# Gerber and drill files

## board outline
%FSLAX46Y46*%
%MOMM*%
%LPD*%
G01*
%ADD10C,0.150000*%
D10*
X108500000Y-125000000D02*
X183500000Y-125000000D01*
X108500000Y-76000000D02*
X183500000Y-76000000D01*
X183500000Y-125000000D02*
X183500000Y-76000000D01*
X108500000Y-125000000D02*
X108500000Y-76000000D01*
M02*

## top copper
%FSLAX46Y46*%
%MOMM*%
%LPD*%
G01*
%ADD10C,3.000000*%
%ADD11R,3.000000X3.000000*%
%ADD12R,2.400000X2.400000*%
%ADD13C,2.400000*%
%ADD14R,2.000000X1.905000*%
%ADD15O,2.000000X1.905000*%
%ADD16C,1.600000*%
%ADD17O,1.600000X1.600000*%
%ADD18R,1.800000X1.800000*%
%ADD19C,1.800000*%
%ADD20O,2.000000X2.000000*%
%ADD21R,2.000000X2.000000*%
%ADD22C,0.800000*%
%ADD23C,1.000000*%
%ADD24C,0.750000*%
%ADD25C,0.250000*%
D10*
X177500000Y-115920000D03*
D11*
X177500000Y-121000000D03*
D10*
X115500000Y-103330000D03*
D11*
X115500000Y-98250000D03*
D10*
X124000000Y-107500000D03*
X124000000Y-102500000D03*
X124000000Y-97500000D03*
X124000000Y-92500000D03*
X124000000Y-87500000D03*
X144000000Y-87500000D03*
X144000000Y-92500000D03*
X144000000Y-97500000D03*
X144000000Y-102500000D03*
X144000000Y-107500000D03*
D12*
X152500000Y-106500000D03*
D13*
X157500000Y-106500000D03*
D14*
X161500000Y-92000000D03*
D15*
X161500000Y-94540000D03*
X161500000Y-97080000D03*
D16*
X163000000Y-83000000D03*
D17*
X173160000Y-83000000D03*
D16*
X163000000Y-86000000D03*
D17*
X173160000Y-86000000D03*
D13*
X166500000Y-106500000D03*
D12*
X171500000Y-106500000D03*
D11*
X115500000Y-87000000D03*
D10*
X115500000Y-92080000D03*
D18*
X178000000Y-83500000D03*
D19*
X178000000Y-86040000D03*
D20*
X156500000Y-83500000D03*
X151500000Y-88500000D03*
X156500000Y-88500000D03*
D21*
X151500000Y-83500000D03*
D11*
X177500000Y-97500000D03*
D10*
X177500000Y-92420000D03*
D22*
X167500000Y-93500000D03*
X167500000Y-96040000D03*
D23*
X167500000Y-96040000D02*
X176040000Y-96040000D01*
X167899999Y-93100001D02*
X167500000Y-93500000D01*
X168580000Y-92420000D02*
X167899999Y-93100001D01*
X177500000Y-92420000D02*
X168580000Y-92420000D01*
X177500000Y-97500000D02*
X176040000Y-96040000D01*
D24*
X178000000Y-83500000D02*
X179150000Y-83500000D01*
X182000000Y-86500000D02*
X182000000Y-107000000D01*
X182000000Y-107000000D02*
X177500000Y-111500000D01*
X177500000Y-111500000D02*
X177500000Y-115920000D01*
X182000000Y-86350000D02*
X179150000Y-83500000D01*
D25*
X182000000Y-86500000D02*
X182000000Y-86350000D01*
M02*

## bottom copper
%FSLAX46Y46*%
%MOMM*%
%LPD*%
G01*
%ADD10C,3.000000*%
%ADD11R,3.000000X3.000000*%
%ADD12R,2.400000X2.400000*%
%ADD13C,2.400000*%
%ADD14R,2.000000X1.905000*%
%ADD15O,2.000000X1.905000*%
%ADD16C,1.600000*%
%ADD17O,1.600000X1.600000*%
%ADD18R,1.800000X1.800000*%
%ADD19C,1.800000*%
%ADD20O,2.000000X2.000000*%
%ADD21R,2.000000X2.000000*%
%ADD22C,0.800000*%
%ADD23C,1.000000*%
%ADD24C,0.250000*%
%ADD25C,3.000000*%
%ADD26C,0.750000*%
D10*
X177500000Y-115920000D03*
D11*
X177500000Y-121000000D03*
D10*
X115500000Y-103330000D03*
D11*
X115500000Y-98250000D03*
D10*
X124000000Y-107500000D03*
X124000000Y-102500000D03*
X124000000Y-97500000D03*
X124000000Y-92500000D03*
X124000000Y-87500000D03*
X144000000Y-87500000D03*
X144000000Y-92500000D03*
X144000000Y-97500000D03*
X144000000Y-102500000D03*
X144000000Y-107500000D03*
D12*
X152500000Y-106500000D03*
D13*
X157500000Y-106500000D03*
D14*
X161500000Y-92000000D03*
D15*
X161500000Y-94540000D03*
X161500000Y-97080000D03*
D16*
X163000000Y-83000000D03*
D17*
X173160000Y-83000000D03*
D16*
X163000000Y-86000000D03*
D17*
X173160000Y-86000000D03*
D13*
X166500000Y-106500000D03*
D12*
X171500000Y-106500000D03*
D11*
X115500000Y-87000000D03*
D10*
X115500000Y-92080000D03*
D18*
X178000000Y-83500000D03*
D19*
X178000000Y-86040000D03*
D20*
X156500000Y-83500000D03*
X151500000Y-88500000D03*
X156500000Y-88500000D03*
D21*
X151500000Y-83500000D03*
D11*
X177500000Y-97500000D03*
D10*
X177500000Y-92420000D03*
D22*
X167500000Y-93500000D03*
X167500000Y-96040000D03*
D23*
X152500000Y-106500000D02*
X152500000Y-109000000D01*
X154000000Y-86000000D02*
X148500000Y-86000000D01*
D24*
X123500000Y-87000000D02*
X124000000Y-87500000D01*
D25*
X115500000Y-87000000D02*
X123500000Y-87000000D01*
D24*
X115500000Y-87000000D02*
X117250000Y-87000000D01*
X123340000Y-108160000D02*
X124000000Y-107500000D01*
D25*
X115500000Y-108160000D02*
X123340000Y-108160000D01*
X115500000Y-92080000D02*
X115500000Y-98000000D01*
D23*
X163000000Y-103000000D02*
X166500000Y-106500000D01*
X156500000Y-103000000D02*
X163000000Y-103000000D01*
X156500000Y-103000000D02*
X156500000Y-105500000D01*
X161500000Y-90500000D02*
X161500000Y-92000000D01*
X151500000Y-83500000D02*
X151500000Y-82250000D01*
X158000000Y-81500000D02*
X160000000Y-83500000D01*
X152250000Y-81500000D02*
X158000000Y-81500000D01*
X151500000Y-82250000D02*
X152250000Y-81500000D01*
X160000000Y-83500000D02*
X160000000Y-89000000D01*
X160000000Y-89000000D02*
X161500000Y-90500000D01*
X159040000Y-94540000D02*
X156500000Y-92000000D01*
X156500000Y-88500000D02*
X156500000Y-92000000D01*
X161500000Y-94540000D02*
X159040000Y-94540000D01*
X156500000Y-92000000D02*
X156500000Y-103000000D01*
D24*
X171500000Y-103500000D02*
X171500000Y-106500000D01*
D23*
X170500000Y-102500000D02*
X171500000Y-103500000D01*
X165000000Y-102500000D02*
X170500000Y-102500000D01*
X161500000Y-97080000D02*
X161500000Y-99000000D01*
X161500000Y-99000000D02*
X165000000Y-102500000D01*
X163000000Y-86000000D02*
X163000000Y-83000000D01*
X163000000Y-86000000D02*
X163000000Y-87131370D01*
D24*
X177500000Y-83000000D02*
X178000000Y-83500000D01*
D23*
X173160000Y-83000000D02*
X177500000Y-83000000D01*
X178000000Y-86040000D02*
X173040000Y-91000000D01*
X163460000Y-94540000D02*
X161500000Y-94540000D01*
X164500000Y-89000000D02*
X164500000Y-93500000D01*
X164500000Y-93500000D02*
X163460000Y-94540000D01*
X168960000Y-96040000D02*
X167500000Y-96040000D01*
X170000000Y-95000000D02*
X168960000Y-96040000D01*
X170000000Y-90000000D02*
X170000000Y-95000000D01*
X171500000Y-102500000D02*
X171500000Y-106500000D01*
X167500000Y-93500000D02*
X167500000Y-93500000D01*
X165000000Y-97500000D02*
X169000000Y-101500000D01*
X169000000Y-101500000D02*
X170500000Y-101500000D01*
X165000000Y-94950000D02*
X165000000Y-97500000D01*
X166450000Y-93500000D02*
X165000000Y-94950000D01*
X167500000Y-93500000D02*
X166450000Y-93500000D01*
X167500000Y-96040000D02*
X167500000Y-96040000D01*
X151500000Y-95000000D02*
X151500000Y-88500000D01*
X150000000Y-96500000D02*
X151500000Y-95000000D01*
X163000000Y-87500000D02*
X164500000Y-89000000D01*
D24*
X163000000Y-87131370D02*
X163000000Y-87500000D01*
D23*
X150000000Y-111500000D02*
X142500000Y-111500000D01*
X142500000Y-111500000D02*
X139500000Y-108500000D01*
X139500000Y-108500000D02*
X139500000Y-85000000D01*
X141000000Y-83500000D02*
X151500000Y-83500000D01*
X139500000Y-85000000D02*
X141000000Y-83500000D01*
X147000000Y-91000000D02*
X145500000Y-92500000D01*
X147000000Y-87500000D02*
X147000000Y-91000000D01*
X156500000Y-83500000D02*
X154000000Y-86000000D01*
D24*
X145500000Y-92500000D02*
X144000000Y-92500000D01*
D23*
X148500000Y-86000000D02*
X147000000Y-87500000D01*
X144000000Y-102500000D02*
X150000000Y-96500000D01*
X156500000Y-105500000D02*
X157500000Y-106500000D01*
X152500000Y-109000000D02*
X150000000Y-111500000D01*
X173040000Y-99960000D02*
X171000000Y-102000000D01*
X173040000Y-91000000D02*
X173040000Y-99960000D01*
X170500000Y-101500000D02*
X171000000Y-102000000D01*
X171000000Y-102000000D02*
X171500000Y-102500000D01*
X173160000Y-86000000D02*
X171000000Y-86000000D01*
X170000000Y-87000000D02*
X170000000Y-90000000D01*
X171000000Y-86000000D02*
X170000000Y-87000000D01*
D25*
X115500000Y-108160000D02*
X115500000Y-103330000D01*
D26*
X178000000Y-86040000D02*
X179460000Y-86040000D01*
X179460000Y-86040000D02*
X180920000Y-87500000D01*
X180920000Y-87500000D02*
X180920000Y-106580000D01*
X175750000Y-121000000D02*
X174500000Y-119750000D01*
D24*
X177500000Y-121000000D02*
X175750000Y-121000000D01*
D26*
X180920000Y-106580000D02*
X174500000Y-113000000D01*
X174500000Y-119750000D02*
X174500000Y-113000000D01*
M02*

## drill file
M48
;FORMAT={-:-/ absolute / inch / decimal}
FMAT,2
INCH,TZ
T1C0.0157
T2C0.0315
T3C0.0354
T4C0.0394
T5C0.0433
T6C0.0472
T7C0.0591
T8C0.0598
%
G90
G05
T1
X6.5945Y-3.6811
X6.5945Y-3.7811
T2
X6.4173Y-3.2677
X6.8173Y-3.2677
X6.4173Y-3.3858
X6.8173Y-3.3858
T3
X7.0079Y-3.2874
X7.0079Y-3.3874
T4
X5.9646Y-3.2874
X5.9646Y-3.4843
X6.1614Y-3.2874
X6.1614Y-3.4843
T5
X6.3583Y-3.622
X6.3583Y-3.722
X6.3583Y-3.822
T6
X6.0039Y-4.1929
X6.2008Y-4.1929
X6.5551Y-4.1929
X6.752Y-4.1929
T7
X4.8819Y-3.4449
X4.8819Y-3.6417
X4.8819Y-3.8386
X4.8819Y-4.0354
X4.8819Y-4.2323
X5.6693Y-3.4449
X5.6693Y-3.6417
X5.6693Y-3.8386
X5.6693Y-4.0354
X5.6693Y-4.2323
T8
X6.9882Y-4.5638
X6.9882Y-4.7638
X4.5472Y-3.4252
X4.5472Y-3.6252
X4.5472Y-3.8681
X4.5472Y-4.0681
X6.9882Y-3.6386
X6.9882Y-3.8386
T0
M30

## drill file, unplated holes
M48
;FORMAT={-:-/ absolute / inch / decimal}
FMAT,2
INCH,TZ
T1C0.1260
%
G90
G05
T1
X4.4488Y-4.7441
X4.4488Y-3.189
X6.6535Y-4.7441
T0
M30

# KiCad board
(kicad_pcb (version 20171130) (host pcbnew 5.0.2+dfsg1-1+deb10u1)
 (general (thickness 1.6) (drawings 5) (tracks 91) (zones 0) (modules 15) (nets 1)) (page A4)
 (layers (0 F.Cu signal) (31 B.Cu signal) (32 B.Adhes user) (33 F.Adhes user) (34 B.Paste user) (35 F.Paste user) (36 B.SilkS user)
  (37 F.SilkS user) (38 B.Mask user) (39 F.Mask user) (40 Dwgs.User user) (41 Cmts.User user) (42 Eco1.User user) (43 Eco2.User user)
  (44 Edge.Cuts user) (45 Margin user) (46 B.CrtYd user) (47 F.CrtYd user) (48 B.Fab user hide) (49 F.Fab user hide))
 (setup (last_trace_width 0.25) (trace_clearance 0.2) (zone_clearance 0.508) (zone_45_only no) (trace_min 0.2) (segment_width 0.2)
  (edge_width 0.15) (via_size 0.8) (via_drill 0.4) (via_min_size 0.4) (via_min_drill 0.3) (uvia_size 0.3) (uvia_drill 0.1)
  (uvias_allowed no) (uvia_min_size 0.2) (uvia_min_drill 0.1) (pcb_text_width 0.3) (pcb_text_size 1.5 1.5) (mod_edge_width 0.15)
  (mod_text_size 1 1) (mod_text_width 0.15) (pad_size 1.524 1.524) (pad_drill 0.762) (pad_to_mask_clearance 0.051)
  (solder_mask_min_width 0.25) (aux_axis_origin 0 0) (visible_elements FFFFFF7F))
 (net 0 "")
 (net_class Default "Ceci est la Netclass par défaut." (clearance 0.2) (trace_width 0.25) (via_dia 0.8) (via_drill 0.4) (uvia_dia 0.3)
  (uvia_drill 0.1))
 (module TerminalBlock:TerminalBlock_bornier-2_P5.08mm (layer F.Cu) (at 177.5 121 90)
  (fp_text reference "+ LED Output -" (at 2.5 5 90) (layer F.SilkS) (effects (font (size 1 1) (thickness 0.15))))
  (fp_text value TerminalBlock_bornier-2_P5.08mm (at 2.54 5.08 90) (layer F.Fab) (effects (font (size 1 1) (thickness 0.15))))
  (pad 2 thru_hole circle (at 5.08 0 90) (size 3 3) (drill 1.52) (layers *.Cu *.Mask))
  (pad 1 thru_hole rect (at 0 0 90) (size 3 3) (drill 1.52) (layers *.Cu *.Mask)))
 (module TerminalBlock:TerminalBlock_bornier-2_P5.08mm (layer F.Cu) (at 115.5 98.25 270)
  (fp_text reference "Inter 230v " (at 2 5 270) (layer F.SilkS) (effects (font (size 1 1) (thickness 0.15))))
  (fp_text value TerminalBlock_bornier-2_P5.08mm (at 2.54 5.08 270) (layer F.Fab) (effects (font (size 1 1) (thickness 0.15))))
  (pad 2 thru_hole circle (at 5.08 0 270) (size 3 3) (drill 1.52) (layers *.Cu *.Mask))
  (pad 1 thru_hole rect (at 0 0 270) (size 3 3) (drill 1.52) (layers *.Cu *.Mask)))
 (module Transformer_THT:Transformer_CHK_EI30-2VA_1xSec (layer F.Cu) (at 124 107.5)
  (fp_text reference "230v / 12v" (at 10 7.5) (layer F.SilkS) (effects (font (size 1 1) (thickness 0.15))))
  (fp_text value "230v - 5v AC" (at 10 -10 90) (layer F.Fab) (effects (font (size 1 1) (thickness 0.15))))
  (pad 1 thru_hole circle (at 0 0) (size 3 3) (drill 1.5) (layers *.Cu *.Mask))
  (pad 2 thru_hole circle (at 0 -5) (size 3 3) (drill 1.5) (layers *.Cu *.Mask))
  (pad 3 thru_hole circle (at 0 -10) (size 3 3) (drill 1.5) (layers *.Cu *.Mask))
  (pad 4 thru_hole circle (at 0 -15) (size 3 3) (drill 1.5) (layers *.Cu *.Mask))
  (pad 5 thru_hole circle (at 0 -20) (size 3 3) (drill 1.5) (layers *.Cu *.Mask))
  (pad 6 thru_hole circle (at 20 -20) (size 3 3) (drill 1.5) (layers *.Cu *.Mask))
  (pad 7 thru_hole circle (at 20 -15) (size 3 3) (drill 1.5) (layers *.Cu *.Mask))
  (pad 8 thru_hole circle (at 20 -10) (size 3 3) (drill 1.5) (layers *.Cu *.Mask))
  (pad 9 thru_hole circle (at 20 -5) (size 3 3) (drill 1.5) (layers *.Cu *.Mask))
  (pad 10 thru_hole circle (at 20 0) (size 3 3) (drill 1.5) (layers *.Cu *.Mask)))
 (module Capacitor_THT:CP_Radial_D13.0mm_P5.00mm (layer F.Cu) (at 152.5 106.5)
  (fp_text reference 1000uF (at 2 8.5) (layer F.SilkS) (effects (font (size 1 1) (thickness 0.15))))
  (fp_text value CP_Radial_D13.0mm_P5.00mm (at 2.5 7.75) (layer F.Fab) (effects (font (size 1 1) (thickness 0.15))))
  (pad 1 thru_hole rect (at 0 0) (size 2.4 2.4) (drill 1.2) (layers *.Cu *.Mask))
  (pad 2 thru_hole circle (at 5 0) (size 2.4 2.4) (drill 1.2) (layers *.Cu *.Mask)))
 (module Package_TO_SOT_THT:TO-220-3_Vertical (layer F.Cu) (at 161.5 92 270)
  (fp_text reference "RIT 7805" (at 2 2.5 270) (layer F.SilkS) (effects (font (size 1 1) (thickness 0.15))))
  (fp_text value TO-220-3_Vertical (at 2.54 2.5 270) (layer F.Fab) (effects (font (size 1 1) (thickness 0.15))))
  (pad 1 thru_hole rect (at 0 0 270) (size 1.905 2) (drill 1.1) (layers *.Cu *.Mask))
  (pad 2 thru_hole oval (at 2.54 0 270) (size 1.905 2) (drill 1.1) (layers *.Cu *.Mask))
  (pad 3 thru_hole oval (at 5.08 0 270) (size 1.905 2) (drill 1.1) (layers *.Cu *.Mask)))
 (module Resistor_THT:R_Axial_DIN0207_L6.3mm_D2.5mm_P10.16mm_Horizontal (layer F.Cu) (at 163 83)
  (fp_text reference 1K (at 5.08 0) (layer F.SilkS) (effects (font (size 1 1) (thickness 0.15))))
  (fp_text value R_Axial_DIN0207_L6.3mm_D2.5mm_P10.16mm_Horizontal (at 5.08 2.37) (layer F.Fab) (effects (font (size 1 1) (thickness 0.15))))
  (pad 1 thru_hole circle (at 0 0) (size 1.6 1.6) (drill 0.8) (layers *.Cu *.Mask))
  (pad 2 thru_hole oval (at 10.16 0) (size 1.6 1.6) (drill 0.8) (layers *.Cu *.Mask)))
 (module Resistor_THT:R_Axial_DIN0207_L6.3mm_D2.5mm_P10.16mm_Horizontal (layer F.Cu) (at 163 86)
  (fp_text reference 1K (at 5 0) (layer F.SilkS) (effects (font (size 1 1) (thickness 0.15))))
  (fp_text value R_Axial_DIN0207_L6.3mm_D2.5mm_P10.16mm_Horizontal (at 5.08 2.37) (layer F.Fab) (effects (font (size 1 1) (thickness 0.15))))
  (pad 1 thru_hole circle (at 0 0) (size 1.6 1.6) (drill 0.8) (layers *.Cu *.Mask))
  (pad 2 thru_hole oval (at 10.16 0) (size 1.6 1.6) (drill 0.8) (layers *.Cu *.Mask)))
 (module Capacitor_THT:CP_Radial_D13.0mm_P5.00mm (layer F.Cu) (at 171.5 106.5 180)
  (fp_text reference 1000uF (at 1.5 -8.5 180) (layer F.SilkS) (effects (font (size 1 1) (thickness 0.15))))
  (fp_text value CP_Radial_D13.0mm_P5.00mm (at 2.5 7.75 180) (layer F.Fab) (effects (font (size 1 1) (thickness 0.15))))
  (pad 2 thru_hole circle (at 5 0 180) (size 2.4 2.4) (drill 1.2) (layers *.Cu *.Mask))
  (pad 1 thru_hole rect (at 0 0 180) (size 2.4 2.4) (drill 1.2) (layers *.Cu *.Mask)))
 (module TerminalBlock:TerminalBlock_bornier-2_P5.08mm (layer F.Cu) (at 115.5 87 270)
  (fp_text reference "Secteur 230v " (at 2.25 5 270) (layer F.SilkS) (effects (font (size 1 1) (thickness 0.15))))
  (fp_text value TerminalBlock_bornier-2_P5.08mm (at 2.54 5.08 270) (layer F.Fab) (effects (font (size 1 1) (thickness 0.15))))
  (pad 1 thru_hole rect (at 0 0 270) (size 3 3) (drill 1.52) (layers *.Cu *.Mask))
  (pad 2 thru_hole circle (at 5.08 0 270) (size 3 3) (drill 1.52) (layers *.Cu *.Mask)))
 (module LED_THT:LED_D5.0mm (layer F.Cu) (at 178 83.5 270)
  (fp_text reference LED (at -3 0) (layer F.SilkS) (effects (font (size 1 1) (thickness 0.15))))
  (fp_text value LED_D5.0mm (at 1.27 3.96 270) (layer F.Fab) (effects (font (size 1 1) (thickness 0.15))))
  (pad 1 thru_hole rect (at 0 0 270) (size 1.8 1.8) (drill 0.9) (layers *.Cu *.Mask))
  (pad 2 thru_hole circle (at 2.54 0 270) (size 1.8 1.8) (drill 0.9) (layers *.Cu *.Mask)))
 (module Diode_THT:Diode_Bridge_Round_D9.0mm (layer F.Cu) (at 151.5 83.5)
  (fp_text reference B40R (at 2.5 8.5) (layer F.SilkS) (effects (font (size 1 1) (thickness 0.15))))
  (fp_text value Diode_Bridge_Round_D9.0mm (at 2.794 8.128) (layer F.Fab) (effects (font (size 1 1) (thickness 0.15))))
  (pad 4 thru_hole oval (at 5 0) (size 2 2) (drill 1) (layers *.Cu *.Mask))
  (pad 2 thru_hole oval (at 0 5) (size 2 2) (drill 1) (layers *.Cu *.Mask))
  (pad 3 thru_hole oval (at 5 5) (size 2 2) (drill 1) (layers *.Cu *.Mask))
  (pad 1 thru_hole rect (at 0 0) (size 2 2) (drill 1) (layers *.Cu *.Mask)))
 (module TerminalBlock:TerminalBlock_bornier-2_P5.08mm (layer F.Cu) (at 177.5 97.5 90)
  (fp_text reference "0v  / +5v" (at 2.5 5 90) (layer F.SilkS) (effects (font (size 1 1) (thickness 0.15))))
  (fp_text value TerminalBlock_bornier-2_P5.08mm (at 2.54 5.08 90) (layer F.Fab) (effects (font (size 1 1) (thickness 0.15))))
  (pad 1 thru_hole rect (at 0 0 90) (size 3 3) (drill 1.52) (layers *.Cu *.Mask))
  (pad 2 thru_hole circle (at 5.08 0 90) (size 3 3) (drill 1.52) (layers *.Cu *.Mask)))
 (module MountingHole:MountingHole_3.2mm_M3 (layer F.Cu) (at 113 120.5)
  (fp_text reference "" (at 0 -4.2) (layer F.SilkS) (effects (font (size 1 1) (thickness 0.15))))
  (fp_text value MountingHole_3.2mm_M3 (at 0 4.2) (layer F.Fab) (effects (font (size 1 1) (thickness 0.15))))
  (pad 1 np_thru_hole circle (at 0 0) (size 3.2 3.2) (drill 3.2) (layers *.Cu *.Mask)))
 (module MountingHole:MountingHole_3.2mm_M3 (layer F.Cu) (at 113 81)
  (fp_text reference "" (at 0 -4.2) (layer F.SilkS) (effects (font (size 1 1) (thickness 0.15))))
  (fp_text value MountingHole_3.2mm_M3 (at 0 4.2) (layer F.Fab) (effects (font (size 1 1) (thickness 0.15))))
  (pad 1 np_thru_hole circle (at 0 0) (size 3.2 3.2) (drill 3.2) (layers *.Cu *.Mask)))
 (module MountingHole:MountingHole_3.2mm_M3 (layer F.Cu) (at 169 120.5)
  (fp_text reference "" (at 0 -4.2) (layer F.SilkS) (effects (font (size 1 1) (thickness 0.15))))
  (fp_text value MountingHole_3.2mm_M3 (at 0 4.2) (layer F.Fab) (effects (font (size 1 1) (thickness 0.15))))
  (pad 1 np_thru_hole circle (at 0 0) (size 3.2 3.2) (drill 3.2) (layers *.Cu *.Mask)))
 (gr_line (start 108.5 125) (end 183.5 125) (layer Edge.Cuts) (width 0.15))
 (gr_line (start 108.5 76) (end 183.5 76) (layer Edge.Cuts) (width 0.15))
 (gr_line (start 183.5 125) (end 183.5 76) (layer Edge.Cuts) (width 0.15))
 (gr_line (start 108.5 125) (end 108.5 76) (layer Edge.Cuts) (width 0.15))
 (segment (start 152.5 106.5) (end 152.5 109) (width 1) (layer B.Cu) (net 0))
 (segment (start 154 86) (end 148.5 86) (width 1) (layer B.Cu) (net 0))
 (segment (start 123.5 87) (end 124 87.5) (width 0.25) (layer B.Cu) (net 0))
 (segment (start 115.5 87) (end 123.5 87) (width 3) (layer B.Cu) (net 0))
 (segment (start 115.5 87) (end 117.25 87) (width 0.25) (layer B.Cu) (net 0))
 (segment (start 123.34 108.16) (end 124 107.5) (width 0.25) (layer B.Cu) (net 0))
 (segment (start 115.5 108.16) (end 123.34 108.16) (width 3) (layer B.Cu) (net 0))
 (segment (start 115.5 92.08) (end 115.5 98) (width 3) (layer B.Cu) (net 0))
 (segment (start 163 103) (end 166.5 106.5) (width 1) (layer B.Cu) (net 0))
 (segment (start 156.5 103) (end 163 103) (width 1) (layer B.Cu) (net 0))
 (segment (start 156.5 103) (end 156.5 105.5) (width 1) (layer B.Cu) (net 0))
 (segment (start 161.5 90.5) (end 161.5 92) (width 1) (layer B.Cu) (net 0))
 (segment (start 151.5 83.5) (end 151.5 82.25) (width 1) (layer B.Cu) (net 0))
 (segment (start 158 81.5) (end 160 83.5) (width 1) (layer B.Cu) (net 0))
 (segment (start 152.25 81.5) (end 158 81.5) (width 1) (layer B.Cu) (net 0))
 (segment (start 151.5 82.25) (end 152.25 81.5) (width 1) (layer B.Cu) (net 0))
 (segment (start 160 83.5) (end 160 89) (width 1) (layer B.Cu) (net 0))
 (segment (start 160 89) (end 161.5 90.5) (width 1) (layer B.Cu) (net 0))
 (segment (start 159.04 94.54) (end 156.5 92) (width 1) (layer B.Cu) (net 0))
 (segment (start 156.5 88.5) (end 156.5 92) (width 1) (layer B.Cu) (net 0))
 (segment (start 161.5 94.54) (end 159.04 94.54) (width 1) (layer B.Cu) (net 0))
 (segment (start 156.5 92) (end 156.5 103) (width 1) (layer B.Cu) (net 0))
 (segment (start 171.5 103.5) (end 171.5 106.5) (width 0.25) (layer B.Cu) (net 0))
 (segment (start 170.5 102.5) (end 171.5 103.5) (width 1) (layer B.Cu) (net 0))
 (segment (start 165 102.5) (end 170.5 102.5) (width 1) (layer B.Cu) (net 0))
 (segment (start 161.5 97.08) (end 161.5 99) (width 1) (layer B.Cu) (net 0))
 (segment (start 161.5 99) (end 165 102.5) (width 1) (layer B.Cu) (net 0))
 (segment (start 163 86) (end 163 83) (width 1) (layer B.Cu) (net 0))
 (segment (start 163 86) (end 163 87.13137) (width 1) (layer B.Cu) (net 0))
 (segment (start 177.5 83) (end 178 83.5) (width 0.25) (layer B.Cu) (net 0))
 (segment (start 173.16 83) (end 177.5 83) (width 1) (layer B.Cu) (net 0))
 (segment (start 178 86.04) (end 173.04 91) (width 1) (layer B.Cu) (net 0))
 (segment (start 163.46 94.54) (end 161.5 94.54) (width 1) (layer B.Cu) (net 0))
 (segment (start 164.5 89) (end 164.5 93.5) (width 1) (layer B.Cu) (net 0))
 (segment (start 164.5 93.5) (end 163.46 94.54) (width 1) (layer B.Cu) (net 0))
 (segment (start 168.96 96.04) (end 167.5 96.04) (width 1) (layer B.Cu) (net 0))
 (segment (start 170 95) (end 168.96 96.04) (width 1) (layer B.Cu) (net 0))
 (segment (start 170 90) (end 170 95) (width 1) (layer B.Cu) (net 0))
 (segment (start 171.5 102.5) (end 171.5 106.5) (width 1) (layer B.Cu) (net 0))
 (segment (start 167.5 93.5) (end 167.5 93.5) (width 1) (layer B.Cu) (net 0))
 (segment (start 165 97.5) (end 169 101.5) (width 1) (layer B.Cu) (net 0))
 (segment (start 169 101.5) (end 170.5 101.5) (width 1) (layer B.Cu) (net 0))
 (segment (start 165 94.95) (end 165 97.5) (width 1) (layer B.Cu) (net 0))
 (segment (start 166.45 93.5) (end 165 94.95) (width 1) (layer B.Cu) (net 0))
 (segment (start 167.5 93.5) (end 166.45 93.5) (width 1) (layer B.Cu) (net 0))
 (via (at 167.5 93.5) (size 0.8) (drill 0.4) (layers F.Cu B.Cu) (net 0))
 (segment (start 167.5 96.04) (end 167.5 96.04) (width 1) (layer B.Cu) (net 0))
 (via (at 167.5 96.04) (size 0.8) (drill 0.4) (layers F.Cu B.Cu) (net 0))
 (segment (start 151.5 95) (end 151.5 88.5) (width 1) (layer B.Cu) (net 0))
 (segment (start 150 96.5) (end 151.5 95) (width 1) (layer B.Cu) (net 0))
 (segment (start 163 87.5) (end 164.5 89) (width 1) (layer B.Cu) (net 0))
 (segment (start 163 87.13137) (end 163 87.5) (width 0.25) (layer B.Cu) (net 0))
 (segment (start 150 111.5) (end 142.5 111.5) (width 1) (layer B.Cu) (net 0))
 (segment (start 142.5 111.5) (end 139.5 108.5) (width 1) (layer B.Cu) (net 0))
 (segment (start 139.5 108.5) (end 139.5 85) (width 1) (layer B.Cu) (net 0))
 (segment (start 141 83.5) (end 151.5 83.5) (width 1) (layer B.Cu) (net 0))
 (segment (start 139.5 85) (end 141 83.5) (width 1) (layer B.Cu) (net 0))
 (segment (start 147 91) (end 145.5 92.5) (width 1) (layer B.Cu) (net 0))
 (segment (start 147 87.5) (end 147 91) (width 1) (layer B.Cu) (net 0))
 (segment (start 156.5 83.5) (end 154 86) (width 1) (layer B.Cu) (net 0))
 (segment (start 145.5 92.5) (end 144 92.5) (width 0.25) (layer B.Cu) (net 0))
 (segment (start 148.5 86) (end 147 87.5) (width 1) (layer B.Cu) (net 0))
 (segment (start 144 102.5) (end 150 96.5) (width 1) (layer B.Cu) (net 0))
 (segment (start 156.5 105.5) (end 157.5 106.5) (width 1) (layer B.Cu) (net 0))
 (segment (start 152.5 109) (end 150 111.5) (width 1) (layer B.Cu) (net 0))
 (segment (start 173.04 99.96) (end 171 102) (width 1) (layer B.Cu) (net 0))
 (segment (start 173.04 91) (end 173.04 99.96) (width 1) (layer B.Cu) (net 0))
 (segment (start 170.5 101.5) (end 171 102) (width 1) (layer B.Cu) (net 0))
 (segment (start 171 102) (end 171.5 102.5) (width 1) (layer B.Cu) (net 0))
 (segment (start 173.16 86) (end 171 86) (width 1) (layer B.Cu) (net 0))
 (segment (start 170 87) (end 170 90) (width 1) (layer B.Cu) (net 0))
 (segment (start 171 86) (end 170 87) (width 1) (layer B.Cu) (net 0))
 (segment (start 167.5 96.04) (end 176.04 96.04) (width 1) (layer F.Cu) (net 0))
 (segment (start 167.899999 93.100001) (end 167.5 93.5) (width 1) (layer F.Cu) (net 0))
 (segment (start 168.58 92.42) (end 167.899999 93.100001) (width 1) (layer F.Cu) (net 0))
 (segment (start 177.5 92.42) (end 168.58 92.42) (width 1) (layer F.Cu) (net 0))
 (segment (start 177.5 97.5) (end 176.04 96.04) (width 1) (layer F.Cu) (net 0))
 (segment (start 115.5 108.16) (end 115.5 103.33) (width 3) (layer B.Cu) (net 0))
 (segment (start 178 86.04) (end 179.46 86.04) (width 0.75) (layer B.Cu) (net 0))
 (segment (start 179.46 86.04) (end 180.92 87.5) (width 0.75) (layer B.Cu) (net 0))
 (segment (start 180.92 87.5) (end 180.92 106.58) (width 0.75) (layer B.Cu) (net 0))
 (segment (start 178 83.5) (end 179.15 83.5) (width 0.75) (layer F.Cu) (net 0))
 (segment (start 182 86.5) (end 182 107) (width 0.75) (layer F.Cu) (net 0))
 (segment (start 182 107) (end 177.5 111.5) (width 0.75) (layer F.Cu) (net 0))
 (segment (start 177.5 111.5) (end 177.5 115.92) (width 0.75) (layer F.Cu) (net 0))
 (segment (start 175.75 121) (end 174.5 119.75) (width 0.75) (layer B.Cu) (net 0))
 (segment (start 177.5 121) (end 175.75 121) (width 0.25) (layer B.Cu) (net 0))
 (segment (start 180.92 106.58) (end 174.5 113) (width 0.75) (layer B.Cu) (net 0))
 (segment (start 174.5 119.75) (end 174.5 113) (width 0.75) (layer B.Cu) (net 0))
 (segment (start 182 86.35) (end 179.15 83.5) (width 0.75) (layer F.Cu) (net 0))
 (segment (start 182 86.5) (end 182 86.35) (width 0.25) (layer F.Cu) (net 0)))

